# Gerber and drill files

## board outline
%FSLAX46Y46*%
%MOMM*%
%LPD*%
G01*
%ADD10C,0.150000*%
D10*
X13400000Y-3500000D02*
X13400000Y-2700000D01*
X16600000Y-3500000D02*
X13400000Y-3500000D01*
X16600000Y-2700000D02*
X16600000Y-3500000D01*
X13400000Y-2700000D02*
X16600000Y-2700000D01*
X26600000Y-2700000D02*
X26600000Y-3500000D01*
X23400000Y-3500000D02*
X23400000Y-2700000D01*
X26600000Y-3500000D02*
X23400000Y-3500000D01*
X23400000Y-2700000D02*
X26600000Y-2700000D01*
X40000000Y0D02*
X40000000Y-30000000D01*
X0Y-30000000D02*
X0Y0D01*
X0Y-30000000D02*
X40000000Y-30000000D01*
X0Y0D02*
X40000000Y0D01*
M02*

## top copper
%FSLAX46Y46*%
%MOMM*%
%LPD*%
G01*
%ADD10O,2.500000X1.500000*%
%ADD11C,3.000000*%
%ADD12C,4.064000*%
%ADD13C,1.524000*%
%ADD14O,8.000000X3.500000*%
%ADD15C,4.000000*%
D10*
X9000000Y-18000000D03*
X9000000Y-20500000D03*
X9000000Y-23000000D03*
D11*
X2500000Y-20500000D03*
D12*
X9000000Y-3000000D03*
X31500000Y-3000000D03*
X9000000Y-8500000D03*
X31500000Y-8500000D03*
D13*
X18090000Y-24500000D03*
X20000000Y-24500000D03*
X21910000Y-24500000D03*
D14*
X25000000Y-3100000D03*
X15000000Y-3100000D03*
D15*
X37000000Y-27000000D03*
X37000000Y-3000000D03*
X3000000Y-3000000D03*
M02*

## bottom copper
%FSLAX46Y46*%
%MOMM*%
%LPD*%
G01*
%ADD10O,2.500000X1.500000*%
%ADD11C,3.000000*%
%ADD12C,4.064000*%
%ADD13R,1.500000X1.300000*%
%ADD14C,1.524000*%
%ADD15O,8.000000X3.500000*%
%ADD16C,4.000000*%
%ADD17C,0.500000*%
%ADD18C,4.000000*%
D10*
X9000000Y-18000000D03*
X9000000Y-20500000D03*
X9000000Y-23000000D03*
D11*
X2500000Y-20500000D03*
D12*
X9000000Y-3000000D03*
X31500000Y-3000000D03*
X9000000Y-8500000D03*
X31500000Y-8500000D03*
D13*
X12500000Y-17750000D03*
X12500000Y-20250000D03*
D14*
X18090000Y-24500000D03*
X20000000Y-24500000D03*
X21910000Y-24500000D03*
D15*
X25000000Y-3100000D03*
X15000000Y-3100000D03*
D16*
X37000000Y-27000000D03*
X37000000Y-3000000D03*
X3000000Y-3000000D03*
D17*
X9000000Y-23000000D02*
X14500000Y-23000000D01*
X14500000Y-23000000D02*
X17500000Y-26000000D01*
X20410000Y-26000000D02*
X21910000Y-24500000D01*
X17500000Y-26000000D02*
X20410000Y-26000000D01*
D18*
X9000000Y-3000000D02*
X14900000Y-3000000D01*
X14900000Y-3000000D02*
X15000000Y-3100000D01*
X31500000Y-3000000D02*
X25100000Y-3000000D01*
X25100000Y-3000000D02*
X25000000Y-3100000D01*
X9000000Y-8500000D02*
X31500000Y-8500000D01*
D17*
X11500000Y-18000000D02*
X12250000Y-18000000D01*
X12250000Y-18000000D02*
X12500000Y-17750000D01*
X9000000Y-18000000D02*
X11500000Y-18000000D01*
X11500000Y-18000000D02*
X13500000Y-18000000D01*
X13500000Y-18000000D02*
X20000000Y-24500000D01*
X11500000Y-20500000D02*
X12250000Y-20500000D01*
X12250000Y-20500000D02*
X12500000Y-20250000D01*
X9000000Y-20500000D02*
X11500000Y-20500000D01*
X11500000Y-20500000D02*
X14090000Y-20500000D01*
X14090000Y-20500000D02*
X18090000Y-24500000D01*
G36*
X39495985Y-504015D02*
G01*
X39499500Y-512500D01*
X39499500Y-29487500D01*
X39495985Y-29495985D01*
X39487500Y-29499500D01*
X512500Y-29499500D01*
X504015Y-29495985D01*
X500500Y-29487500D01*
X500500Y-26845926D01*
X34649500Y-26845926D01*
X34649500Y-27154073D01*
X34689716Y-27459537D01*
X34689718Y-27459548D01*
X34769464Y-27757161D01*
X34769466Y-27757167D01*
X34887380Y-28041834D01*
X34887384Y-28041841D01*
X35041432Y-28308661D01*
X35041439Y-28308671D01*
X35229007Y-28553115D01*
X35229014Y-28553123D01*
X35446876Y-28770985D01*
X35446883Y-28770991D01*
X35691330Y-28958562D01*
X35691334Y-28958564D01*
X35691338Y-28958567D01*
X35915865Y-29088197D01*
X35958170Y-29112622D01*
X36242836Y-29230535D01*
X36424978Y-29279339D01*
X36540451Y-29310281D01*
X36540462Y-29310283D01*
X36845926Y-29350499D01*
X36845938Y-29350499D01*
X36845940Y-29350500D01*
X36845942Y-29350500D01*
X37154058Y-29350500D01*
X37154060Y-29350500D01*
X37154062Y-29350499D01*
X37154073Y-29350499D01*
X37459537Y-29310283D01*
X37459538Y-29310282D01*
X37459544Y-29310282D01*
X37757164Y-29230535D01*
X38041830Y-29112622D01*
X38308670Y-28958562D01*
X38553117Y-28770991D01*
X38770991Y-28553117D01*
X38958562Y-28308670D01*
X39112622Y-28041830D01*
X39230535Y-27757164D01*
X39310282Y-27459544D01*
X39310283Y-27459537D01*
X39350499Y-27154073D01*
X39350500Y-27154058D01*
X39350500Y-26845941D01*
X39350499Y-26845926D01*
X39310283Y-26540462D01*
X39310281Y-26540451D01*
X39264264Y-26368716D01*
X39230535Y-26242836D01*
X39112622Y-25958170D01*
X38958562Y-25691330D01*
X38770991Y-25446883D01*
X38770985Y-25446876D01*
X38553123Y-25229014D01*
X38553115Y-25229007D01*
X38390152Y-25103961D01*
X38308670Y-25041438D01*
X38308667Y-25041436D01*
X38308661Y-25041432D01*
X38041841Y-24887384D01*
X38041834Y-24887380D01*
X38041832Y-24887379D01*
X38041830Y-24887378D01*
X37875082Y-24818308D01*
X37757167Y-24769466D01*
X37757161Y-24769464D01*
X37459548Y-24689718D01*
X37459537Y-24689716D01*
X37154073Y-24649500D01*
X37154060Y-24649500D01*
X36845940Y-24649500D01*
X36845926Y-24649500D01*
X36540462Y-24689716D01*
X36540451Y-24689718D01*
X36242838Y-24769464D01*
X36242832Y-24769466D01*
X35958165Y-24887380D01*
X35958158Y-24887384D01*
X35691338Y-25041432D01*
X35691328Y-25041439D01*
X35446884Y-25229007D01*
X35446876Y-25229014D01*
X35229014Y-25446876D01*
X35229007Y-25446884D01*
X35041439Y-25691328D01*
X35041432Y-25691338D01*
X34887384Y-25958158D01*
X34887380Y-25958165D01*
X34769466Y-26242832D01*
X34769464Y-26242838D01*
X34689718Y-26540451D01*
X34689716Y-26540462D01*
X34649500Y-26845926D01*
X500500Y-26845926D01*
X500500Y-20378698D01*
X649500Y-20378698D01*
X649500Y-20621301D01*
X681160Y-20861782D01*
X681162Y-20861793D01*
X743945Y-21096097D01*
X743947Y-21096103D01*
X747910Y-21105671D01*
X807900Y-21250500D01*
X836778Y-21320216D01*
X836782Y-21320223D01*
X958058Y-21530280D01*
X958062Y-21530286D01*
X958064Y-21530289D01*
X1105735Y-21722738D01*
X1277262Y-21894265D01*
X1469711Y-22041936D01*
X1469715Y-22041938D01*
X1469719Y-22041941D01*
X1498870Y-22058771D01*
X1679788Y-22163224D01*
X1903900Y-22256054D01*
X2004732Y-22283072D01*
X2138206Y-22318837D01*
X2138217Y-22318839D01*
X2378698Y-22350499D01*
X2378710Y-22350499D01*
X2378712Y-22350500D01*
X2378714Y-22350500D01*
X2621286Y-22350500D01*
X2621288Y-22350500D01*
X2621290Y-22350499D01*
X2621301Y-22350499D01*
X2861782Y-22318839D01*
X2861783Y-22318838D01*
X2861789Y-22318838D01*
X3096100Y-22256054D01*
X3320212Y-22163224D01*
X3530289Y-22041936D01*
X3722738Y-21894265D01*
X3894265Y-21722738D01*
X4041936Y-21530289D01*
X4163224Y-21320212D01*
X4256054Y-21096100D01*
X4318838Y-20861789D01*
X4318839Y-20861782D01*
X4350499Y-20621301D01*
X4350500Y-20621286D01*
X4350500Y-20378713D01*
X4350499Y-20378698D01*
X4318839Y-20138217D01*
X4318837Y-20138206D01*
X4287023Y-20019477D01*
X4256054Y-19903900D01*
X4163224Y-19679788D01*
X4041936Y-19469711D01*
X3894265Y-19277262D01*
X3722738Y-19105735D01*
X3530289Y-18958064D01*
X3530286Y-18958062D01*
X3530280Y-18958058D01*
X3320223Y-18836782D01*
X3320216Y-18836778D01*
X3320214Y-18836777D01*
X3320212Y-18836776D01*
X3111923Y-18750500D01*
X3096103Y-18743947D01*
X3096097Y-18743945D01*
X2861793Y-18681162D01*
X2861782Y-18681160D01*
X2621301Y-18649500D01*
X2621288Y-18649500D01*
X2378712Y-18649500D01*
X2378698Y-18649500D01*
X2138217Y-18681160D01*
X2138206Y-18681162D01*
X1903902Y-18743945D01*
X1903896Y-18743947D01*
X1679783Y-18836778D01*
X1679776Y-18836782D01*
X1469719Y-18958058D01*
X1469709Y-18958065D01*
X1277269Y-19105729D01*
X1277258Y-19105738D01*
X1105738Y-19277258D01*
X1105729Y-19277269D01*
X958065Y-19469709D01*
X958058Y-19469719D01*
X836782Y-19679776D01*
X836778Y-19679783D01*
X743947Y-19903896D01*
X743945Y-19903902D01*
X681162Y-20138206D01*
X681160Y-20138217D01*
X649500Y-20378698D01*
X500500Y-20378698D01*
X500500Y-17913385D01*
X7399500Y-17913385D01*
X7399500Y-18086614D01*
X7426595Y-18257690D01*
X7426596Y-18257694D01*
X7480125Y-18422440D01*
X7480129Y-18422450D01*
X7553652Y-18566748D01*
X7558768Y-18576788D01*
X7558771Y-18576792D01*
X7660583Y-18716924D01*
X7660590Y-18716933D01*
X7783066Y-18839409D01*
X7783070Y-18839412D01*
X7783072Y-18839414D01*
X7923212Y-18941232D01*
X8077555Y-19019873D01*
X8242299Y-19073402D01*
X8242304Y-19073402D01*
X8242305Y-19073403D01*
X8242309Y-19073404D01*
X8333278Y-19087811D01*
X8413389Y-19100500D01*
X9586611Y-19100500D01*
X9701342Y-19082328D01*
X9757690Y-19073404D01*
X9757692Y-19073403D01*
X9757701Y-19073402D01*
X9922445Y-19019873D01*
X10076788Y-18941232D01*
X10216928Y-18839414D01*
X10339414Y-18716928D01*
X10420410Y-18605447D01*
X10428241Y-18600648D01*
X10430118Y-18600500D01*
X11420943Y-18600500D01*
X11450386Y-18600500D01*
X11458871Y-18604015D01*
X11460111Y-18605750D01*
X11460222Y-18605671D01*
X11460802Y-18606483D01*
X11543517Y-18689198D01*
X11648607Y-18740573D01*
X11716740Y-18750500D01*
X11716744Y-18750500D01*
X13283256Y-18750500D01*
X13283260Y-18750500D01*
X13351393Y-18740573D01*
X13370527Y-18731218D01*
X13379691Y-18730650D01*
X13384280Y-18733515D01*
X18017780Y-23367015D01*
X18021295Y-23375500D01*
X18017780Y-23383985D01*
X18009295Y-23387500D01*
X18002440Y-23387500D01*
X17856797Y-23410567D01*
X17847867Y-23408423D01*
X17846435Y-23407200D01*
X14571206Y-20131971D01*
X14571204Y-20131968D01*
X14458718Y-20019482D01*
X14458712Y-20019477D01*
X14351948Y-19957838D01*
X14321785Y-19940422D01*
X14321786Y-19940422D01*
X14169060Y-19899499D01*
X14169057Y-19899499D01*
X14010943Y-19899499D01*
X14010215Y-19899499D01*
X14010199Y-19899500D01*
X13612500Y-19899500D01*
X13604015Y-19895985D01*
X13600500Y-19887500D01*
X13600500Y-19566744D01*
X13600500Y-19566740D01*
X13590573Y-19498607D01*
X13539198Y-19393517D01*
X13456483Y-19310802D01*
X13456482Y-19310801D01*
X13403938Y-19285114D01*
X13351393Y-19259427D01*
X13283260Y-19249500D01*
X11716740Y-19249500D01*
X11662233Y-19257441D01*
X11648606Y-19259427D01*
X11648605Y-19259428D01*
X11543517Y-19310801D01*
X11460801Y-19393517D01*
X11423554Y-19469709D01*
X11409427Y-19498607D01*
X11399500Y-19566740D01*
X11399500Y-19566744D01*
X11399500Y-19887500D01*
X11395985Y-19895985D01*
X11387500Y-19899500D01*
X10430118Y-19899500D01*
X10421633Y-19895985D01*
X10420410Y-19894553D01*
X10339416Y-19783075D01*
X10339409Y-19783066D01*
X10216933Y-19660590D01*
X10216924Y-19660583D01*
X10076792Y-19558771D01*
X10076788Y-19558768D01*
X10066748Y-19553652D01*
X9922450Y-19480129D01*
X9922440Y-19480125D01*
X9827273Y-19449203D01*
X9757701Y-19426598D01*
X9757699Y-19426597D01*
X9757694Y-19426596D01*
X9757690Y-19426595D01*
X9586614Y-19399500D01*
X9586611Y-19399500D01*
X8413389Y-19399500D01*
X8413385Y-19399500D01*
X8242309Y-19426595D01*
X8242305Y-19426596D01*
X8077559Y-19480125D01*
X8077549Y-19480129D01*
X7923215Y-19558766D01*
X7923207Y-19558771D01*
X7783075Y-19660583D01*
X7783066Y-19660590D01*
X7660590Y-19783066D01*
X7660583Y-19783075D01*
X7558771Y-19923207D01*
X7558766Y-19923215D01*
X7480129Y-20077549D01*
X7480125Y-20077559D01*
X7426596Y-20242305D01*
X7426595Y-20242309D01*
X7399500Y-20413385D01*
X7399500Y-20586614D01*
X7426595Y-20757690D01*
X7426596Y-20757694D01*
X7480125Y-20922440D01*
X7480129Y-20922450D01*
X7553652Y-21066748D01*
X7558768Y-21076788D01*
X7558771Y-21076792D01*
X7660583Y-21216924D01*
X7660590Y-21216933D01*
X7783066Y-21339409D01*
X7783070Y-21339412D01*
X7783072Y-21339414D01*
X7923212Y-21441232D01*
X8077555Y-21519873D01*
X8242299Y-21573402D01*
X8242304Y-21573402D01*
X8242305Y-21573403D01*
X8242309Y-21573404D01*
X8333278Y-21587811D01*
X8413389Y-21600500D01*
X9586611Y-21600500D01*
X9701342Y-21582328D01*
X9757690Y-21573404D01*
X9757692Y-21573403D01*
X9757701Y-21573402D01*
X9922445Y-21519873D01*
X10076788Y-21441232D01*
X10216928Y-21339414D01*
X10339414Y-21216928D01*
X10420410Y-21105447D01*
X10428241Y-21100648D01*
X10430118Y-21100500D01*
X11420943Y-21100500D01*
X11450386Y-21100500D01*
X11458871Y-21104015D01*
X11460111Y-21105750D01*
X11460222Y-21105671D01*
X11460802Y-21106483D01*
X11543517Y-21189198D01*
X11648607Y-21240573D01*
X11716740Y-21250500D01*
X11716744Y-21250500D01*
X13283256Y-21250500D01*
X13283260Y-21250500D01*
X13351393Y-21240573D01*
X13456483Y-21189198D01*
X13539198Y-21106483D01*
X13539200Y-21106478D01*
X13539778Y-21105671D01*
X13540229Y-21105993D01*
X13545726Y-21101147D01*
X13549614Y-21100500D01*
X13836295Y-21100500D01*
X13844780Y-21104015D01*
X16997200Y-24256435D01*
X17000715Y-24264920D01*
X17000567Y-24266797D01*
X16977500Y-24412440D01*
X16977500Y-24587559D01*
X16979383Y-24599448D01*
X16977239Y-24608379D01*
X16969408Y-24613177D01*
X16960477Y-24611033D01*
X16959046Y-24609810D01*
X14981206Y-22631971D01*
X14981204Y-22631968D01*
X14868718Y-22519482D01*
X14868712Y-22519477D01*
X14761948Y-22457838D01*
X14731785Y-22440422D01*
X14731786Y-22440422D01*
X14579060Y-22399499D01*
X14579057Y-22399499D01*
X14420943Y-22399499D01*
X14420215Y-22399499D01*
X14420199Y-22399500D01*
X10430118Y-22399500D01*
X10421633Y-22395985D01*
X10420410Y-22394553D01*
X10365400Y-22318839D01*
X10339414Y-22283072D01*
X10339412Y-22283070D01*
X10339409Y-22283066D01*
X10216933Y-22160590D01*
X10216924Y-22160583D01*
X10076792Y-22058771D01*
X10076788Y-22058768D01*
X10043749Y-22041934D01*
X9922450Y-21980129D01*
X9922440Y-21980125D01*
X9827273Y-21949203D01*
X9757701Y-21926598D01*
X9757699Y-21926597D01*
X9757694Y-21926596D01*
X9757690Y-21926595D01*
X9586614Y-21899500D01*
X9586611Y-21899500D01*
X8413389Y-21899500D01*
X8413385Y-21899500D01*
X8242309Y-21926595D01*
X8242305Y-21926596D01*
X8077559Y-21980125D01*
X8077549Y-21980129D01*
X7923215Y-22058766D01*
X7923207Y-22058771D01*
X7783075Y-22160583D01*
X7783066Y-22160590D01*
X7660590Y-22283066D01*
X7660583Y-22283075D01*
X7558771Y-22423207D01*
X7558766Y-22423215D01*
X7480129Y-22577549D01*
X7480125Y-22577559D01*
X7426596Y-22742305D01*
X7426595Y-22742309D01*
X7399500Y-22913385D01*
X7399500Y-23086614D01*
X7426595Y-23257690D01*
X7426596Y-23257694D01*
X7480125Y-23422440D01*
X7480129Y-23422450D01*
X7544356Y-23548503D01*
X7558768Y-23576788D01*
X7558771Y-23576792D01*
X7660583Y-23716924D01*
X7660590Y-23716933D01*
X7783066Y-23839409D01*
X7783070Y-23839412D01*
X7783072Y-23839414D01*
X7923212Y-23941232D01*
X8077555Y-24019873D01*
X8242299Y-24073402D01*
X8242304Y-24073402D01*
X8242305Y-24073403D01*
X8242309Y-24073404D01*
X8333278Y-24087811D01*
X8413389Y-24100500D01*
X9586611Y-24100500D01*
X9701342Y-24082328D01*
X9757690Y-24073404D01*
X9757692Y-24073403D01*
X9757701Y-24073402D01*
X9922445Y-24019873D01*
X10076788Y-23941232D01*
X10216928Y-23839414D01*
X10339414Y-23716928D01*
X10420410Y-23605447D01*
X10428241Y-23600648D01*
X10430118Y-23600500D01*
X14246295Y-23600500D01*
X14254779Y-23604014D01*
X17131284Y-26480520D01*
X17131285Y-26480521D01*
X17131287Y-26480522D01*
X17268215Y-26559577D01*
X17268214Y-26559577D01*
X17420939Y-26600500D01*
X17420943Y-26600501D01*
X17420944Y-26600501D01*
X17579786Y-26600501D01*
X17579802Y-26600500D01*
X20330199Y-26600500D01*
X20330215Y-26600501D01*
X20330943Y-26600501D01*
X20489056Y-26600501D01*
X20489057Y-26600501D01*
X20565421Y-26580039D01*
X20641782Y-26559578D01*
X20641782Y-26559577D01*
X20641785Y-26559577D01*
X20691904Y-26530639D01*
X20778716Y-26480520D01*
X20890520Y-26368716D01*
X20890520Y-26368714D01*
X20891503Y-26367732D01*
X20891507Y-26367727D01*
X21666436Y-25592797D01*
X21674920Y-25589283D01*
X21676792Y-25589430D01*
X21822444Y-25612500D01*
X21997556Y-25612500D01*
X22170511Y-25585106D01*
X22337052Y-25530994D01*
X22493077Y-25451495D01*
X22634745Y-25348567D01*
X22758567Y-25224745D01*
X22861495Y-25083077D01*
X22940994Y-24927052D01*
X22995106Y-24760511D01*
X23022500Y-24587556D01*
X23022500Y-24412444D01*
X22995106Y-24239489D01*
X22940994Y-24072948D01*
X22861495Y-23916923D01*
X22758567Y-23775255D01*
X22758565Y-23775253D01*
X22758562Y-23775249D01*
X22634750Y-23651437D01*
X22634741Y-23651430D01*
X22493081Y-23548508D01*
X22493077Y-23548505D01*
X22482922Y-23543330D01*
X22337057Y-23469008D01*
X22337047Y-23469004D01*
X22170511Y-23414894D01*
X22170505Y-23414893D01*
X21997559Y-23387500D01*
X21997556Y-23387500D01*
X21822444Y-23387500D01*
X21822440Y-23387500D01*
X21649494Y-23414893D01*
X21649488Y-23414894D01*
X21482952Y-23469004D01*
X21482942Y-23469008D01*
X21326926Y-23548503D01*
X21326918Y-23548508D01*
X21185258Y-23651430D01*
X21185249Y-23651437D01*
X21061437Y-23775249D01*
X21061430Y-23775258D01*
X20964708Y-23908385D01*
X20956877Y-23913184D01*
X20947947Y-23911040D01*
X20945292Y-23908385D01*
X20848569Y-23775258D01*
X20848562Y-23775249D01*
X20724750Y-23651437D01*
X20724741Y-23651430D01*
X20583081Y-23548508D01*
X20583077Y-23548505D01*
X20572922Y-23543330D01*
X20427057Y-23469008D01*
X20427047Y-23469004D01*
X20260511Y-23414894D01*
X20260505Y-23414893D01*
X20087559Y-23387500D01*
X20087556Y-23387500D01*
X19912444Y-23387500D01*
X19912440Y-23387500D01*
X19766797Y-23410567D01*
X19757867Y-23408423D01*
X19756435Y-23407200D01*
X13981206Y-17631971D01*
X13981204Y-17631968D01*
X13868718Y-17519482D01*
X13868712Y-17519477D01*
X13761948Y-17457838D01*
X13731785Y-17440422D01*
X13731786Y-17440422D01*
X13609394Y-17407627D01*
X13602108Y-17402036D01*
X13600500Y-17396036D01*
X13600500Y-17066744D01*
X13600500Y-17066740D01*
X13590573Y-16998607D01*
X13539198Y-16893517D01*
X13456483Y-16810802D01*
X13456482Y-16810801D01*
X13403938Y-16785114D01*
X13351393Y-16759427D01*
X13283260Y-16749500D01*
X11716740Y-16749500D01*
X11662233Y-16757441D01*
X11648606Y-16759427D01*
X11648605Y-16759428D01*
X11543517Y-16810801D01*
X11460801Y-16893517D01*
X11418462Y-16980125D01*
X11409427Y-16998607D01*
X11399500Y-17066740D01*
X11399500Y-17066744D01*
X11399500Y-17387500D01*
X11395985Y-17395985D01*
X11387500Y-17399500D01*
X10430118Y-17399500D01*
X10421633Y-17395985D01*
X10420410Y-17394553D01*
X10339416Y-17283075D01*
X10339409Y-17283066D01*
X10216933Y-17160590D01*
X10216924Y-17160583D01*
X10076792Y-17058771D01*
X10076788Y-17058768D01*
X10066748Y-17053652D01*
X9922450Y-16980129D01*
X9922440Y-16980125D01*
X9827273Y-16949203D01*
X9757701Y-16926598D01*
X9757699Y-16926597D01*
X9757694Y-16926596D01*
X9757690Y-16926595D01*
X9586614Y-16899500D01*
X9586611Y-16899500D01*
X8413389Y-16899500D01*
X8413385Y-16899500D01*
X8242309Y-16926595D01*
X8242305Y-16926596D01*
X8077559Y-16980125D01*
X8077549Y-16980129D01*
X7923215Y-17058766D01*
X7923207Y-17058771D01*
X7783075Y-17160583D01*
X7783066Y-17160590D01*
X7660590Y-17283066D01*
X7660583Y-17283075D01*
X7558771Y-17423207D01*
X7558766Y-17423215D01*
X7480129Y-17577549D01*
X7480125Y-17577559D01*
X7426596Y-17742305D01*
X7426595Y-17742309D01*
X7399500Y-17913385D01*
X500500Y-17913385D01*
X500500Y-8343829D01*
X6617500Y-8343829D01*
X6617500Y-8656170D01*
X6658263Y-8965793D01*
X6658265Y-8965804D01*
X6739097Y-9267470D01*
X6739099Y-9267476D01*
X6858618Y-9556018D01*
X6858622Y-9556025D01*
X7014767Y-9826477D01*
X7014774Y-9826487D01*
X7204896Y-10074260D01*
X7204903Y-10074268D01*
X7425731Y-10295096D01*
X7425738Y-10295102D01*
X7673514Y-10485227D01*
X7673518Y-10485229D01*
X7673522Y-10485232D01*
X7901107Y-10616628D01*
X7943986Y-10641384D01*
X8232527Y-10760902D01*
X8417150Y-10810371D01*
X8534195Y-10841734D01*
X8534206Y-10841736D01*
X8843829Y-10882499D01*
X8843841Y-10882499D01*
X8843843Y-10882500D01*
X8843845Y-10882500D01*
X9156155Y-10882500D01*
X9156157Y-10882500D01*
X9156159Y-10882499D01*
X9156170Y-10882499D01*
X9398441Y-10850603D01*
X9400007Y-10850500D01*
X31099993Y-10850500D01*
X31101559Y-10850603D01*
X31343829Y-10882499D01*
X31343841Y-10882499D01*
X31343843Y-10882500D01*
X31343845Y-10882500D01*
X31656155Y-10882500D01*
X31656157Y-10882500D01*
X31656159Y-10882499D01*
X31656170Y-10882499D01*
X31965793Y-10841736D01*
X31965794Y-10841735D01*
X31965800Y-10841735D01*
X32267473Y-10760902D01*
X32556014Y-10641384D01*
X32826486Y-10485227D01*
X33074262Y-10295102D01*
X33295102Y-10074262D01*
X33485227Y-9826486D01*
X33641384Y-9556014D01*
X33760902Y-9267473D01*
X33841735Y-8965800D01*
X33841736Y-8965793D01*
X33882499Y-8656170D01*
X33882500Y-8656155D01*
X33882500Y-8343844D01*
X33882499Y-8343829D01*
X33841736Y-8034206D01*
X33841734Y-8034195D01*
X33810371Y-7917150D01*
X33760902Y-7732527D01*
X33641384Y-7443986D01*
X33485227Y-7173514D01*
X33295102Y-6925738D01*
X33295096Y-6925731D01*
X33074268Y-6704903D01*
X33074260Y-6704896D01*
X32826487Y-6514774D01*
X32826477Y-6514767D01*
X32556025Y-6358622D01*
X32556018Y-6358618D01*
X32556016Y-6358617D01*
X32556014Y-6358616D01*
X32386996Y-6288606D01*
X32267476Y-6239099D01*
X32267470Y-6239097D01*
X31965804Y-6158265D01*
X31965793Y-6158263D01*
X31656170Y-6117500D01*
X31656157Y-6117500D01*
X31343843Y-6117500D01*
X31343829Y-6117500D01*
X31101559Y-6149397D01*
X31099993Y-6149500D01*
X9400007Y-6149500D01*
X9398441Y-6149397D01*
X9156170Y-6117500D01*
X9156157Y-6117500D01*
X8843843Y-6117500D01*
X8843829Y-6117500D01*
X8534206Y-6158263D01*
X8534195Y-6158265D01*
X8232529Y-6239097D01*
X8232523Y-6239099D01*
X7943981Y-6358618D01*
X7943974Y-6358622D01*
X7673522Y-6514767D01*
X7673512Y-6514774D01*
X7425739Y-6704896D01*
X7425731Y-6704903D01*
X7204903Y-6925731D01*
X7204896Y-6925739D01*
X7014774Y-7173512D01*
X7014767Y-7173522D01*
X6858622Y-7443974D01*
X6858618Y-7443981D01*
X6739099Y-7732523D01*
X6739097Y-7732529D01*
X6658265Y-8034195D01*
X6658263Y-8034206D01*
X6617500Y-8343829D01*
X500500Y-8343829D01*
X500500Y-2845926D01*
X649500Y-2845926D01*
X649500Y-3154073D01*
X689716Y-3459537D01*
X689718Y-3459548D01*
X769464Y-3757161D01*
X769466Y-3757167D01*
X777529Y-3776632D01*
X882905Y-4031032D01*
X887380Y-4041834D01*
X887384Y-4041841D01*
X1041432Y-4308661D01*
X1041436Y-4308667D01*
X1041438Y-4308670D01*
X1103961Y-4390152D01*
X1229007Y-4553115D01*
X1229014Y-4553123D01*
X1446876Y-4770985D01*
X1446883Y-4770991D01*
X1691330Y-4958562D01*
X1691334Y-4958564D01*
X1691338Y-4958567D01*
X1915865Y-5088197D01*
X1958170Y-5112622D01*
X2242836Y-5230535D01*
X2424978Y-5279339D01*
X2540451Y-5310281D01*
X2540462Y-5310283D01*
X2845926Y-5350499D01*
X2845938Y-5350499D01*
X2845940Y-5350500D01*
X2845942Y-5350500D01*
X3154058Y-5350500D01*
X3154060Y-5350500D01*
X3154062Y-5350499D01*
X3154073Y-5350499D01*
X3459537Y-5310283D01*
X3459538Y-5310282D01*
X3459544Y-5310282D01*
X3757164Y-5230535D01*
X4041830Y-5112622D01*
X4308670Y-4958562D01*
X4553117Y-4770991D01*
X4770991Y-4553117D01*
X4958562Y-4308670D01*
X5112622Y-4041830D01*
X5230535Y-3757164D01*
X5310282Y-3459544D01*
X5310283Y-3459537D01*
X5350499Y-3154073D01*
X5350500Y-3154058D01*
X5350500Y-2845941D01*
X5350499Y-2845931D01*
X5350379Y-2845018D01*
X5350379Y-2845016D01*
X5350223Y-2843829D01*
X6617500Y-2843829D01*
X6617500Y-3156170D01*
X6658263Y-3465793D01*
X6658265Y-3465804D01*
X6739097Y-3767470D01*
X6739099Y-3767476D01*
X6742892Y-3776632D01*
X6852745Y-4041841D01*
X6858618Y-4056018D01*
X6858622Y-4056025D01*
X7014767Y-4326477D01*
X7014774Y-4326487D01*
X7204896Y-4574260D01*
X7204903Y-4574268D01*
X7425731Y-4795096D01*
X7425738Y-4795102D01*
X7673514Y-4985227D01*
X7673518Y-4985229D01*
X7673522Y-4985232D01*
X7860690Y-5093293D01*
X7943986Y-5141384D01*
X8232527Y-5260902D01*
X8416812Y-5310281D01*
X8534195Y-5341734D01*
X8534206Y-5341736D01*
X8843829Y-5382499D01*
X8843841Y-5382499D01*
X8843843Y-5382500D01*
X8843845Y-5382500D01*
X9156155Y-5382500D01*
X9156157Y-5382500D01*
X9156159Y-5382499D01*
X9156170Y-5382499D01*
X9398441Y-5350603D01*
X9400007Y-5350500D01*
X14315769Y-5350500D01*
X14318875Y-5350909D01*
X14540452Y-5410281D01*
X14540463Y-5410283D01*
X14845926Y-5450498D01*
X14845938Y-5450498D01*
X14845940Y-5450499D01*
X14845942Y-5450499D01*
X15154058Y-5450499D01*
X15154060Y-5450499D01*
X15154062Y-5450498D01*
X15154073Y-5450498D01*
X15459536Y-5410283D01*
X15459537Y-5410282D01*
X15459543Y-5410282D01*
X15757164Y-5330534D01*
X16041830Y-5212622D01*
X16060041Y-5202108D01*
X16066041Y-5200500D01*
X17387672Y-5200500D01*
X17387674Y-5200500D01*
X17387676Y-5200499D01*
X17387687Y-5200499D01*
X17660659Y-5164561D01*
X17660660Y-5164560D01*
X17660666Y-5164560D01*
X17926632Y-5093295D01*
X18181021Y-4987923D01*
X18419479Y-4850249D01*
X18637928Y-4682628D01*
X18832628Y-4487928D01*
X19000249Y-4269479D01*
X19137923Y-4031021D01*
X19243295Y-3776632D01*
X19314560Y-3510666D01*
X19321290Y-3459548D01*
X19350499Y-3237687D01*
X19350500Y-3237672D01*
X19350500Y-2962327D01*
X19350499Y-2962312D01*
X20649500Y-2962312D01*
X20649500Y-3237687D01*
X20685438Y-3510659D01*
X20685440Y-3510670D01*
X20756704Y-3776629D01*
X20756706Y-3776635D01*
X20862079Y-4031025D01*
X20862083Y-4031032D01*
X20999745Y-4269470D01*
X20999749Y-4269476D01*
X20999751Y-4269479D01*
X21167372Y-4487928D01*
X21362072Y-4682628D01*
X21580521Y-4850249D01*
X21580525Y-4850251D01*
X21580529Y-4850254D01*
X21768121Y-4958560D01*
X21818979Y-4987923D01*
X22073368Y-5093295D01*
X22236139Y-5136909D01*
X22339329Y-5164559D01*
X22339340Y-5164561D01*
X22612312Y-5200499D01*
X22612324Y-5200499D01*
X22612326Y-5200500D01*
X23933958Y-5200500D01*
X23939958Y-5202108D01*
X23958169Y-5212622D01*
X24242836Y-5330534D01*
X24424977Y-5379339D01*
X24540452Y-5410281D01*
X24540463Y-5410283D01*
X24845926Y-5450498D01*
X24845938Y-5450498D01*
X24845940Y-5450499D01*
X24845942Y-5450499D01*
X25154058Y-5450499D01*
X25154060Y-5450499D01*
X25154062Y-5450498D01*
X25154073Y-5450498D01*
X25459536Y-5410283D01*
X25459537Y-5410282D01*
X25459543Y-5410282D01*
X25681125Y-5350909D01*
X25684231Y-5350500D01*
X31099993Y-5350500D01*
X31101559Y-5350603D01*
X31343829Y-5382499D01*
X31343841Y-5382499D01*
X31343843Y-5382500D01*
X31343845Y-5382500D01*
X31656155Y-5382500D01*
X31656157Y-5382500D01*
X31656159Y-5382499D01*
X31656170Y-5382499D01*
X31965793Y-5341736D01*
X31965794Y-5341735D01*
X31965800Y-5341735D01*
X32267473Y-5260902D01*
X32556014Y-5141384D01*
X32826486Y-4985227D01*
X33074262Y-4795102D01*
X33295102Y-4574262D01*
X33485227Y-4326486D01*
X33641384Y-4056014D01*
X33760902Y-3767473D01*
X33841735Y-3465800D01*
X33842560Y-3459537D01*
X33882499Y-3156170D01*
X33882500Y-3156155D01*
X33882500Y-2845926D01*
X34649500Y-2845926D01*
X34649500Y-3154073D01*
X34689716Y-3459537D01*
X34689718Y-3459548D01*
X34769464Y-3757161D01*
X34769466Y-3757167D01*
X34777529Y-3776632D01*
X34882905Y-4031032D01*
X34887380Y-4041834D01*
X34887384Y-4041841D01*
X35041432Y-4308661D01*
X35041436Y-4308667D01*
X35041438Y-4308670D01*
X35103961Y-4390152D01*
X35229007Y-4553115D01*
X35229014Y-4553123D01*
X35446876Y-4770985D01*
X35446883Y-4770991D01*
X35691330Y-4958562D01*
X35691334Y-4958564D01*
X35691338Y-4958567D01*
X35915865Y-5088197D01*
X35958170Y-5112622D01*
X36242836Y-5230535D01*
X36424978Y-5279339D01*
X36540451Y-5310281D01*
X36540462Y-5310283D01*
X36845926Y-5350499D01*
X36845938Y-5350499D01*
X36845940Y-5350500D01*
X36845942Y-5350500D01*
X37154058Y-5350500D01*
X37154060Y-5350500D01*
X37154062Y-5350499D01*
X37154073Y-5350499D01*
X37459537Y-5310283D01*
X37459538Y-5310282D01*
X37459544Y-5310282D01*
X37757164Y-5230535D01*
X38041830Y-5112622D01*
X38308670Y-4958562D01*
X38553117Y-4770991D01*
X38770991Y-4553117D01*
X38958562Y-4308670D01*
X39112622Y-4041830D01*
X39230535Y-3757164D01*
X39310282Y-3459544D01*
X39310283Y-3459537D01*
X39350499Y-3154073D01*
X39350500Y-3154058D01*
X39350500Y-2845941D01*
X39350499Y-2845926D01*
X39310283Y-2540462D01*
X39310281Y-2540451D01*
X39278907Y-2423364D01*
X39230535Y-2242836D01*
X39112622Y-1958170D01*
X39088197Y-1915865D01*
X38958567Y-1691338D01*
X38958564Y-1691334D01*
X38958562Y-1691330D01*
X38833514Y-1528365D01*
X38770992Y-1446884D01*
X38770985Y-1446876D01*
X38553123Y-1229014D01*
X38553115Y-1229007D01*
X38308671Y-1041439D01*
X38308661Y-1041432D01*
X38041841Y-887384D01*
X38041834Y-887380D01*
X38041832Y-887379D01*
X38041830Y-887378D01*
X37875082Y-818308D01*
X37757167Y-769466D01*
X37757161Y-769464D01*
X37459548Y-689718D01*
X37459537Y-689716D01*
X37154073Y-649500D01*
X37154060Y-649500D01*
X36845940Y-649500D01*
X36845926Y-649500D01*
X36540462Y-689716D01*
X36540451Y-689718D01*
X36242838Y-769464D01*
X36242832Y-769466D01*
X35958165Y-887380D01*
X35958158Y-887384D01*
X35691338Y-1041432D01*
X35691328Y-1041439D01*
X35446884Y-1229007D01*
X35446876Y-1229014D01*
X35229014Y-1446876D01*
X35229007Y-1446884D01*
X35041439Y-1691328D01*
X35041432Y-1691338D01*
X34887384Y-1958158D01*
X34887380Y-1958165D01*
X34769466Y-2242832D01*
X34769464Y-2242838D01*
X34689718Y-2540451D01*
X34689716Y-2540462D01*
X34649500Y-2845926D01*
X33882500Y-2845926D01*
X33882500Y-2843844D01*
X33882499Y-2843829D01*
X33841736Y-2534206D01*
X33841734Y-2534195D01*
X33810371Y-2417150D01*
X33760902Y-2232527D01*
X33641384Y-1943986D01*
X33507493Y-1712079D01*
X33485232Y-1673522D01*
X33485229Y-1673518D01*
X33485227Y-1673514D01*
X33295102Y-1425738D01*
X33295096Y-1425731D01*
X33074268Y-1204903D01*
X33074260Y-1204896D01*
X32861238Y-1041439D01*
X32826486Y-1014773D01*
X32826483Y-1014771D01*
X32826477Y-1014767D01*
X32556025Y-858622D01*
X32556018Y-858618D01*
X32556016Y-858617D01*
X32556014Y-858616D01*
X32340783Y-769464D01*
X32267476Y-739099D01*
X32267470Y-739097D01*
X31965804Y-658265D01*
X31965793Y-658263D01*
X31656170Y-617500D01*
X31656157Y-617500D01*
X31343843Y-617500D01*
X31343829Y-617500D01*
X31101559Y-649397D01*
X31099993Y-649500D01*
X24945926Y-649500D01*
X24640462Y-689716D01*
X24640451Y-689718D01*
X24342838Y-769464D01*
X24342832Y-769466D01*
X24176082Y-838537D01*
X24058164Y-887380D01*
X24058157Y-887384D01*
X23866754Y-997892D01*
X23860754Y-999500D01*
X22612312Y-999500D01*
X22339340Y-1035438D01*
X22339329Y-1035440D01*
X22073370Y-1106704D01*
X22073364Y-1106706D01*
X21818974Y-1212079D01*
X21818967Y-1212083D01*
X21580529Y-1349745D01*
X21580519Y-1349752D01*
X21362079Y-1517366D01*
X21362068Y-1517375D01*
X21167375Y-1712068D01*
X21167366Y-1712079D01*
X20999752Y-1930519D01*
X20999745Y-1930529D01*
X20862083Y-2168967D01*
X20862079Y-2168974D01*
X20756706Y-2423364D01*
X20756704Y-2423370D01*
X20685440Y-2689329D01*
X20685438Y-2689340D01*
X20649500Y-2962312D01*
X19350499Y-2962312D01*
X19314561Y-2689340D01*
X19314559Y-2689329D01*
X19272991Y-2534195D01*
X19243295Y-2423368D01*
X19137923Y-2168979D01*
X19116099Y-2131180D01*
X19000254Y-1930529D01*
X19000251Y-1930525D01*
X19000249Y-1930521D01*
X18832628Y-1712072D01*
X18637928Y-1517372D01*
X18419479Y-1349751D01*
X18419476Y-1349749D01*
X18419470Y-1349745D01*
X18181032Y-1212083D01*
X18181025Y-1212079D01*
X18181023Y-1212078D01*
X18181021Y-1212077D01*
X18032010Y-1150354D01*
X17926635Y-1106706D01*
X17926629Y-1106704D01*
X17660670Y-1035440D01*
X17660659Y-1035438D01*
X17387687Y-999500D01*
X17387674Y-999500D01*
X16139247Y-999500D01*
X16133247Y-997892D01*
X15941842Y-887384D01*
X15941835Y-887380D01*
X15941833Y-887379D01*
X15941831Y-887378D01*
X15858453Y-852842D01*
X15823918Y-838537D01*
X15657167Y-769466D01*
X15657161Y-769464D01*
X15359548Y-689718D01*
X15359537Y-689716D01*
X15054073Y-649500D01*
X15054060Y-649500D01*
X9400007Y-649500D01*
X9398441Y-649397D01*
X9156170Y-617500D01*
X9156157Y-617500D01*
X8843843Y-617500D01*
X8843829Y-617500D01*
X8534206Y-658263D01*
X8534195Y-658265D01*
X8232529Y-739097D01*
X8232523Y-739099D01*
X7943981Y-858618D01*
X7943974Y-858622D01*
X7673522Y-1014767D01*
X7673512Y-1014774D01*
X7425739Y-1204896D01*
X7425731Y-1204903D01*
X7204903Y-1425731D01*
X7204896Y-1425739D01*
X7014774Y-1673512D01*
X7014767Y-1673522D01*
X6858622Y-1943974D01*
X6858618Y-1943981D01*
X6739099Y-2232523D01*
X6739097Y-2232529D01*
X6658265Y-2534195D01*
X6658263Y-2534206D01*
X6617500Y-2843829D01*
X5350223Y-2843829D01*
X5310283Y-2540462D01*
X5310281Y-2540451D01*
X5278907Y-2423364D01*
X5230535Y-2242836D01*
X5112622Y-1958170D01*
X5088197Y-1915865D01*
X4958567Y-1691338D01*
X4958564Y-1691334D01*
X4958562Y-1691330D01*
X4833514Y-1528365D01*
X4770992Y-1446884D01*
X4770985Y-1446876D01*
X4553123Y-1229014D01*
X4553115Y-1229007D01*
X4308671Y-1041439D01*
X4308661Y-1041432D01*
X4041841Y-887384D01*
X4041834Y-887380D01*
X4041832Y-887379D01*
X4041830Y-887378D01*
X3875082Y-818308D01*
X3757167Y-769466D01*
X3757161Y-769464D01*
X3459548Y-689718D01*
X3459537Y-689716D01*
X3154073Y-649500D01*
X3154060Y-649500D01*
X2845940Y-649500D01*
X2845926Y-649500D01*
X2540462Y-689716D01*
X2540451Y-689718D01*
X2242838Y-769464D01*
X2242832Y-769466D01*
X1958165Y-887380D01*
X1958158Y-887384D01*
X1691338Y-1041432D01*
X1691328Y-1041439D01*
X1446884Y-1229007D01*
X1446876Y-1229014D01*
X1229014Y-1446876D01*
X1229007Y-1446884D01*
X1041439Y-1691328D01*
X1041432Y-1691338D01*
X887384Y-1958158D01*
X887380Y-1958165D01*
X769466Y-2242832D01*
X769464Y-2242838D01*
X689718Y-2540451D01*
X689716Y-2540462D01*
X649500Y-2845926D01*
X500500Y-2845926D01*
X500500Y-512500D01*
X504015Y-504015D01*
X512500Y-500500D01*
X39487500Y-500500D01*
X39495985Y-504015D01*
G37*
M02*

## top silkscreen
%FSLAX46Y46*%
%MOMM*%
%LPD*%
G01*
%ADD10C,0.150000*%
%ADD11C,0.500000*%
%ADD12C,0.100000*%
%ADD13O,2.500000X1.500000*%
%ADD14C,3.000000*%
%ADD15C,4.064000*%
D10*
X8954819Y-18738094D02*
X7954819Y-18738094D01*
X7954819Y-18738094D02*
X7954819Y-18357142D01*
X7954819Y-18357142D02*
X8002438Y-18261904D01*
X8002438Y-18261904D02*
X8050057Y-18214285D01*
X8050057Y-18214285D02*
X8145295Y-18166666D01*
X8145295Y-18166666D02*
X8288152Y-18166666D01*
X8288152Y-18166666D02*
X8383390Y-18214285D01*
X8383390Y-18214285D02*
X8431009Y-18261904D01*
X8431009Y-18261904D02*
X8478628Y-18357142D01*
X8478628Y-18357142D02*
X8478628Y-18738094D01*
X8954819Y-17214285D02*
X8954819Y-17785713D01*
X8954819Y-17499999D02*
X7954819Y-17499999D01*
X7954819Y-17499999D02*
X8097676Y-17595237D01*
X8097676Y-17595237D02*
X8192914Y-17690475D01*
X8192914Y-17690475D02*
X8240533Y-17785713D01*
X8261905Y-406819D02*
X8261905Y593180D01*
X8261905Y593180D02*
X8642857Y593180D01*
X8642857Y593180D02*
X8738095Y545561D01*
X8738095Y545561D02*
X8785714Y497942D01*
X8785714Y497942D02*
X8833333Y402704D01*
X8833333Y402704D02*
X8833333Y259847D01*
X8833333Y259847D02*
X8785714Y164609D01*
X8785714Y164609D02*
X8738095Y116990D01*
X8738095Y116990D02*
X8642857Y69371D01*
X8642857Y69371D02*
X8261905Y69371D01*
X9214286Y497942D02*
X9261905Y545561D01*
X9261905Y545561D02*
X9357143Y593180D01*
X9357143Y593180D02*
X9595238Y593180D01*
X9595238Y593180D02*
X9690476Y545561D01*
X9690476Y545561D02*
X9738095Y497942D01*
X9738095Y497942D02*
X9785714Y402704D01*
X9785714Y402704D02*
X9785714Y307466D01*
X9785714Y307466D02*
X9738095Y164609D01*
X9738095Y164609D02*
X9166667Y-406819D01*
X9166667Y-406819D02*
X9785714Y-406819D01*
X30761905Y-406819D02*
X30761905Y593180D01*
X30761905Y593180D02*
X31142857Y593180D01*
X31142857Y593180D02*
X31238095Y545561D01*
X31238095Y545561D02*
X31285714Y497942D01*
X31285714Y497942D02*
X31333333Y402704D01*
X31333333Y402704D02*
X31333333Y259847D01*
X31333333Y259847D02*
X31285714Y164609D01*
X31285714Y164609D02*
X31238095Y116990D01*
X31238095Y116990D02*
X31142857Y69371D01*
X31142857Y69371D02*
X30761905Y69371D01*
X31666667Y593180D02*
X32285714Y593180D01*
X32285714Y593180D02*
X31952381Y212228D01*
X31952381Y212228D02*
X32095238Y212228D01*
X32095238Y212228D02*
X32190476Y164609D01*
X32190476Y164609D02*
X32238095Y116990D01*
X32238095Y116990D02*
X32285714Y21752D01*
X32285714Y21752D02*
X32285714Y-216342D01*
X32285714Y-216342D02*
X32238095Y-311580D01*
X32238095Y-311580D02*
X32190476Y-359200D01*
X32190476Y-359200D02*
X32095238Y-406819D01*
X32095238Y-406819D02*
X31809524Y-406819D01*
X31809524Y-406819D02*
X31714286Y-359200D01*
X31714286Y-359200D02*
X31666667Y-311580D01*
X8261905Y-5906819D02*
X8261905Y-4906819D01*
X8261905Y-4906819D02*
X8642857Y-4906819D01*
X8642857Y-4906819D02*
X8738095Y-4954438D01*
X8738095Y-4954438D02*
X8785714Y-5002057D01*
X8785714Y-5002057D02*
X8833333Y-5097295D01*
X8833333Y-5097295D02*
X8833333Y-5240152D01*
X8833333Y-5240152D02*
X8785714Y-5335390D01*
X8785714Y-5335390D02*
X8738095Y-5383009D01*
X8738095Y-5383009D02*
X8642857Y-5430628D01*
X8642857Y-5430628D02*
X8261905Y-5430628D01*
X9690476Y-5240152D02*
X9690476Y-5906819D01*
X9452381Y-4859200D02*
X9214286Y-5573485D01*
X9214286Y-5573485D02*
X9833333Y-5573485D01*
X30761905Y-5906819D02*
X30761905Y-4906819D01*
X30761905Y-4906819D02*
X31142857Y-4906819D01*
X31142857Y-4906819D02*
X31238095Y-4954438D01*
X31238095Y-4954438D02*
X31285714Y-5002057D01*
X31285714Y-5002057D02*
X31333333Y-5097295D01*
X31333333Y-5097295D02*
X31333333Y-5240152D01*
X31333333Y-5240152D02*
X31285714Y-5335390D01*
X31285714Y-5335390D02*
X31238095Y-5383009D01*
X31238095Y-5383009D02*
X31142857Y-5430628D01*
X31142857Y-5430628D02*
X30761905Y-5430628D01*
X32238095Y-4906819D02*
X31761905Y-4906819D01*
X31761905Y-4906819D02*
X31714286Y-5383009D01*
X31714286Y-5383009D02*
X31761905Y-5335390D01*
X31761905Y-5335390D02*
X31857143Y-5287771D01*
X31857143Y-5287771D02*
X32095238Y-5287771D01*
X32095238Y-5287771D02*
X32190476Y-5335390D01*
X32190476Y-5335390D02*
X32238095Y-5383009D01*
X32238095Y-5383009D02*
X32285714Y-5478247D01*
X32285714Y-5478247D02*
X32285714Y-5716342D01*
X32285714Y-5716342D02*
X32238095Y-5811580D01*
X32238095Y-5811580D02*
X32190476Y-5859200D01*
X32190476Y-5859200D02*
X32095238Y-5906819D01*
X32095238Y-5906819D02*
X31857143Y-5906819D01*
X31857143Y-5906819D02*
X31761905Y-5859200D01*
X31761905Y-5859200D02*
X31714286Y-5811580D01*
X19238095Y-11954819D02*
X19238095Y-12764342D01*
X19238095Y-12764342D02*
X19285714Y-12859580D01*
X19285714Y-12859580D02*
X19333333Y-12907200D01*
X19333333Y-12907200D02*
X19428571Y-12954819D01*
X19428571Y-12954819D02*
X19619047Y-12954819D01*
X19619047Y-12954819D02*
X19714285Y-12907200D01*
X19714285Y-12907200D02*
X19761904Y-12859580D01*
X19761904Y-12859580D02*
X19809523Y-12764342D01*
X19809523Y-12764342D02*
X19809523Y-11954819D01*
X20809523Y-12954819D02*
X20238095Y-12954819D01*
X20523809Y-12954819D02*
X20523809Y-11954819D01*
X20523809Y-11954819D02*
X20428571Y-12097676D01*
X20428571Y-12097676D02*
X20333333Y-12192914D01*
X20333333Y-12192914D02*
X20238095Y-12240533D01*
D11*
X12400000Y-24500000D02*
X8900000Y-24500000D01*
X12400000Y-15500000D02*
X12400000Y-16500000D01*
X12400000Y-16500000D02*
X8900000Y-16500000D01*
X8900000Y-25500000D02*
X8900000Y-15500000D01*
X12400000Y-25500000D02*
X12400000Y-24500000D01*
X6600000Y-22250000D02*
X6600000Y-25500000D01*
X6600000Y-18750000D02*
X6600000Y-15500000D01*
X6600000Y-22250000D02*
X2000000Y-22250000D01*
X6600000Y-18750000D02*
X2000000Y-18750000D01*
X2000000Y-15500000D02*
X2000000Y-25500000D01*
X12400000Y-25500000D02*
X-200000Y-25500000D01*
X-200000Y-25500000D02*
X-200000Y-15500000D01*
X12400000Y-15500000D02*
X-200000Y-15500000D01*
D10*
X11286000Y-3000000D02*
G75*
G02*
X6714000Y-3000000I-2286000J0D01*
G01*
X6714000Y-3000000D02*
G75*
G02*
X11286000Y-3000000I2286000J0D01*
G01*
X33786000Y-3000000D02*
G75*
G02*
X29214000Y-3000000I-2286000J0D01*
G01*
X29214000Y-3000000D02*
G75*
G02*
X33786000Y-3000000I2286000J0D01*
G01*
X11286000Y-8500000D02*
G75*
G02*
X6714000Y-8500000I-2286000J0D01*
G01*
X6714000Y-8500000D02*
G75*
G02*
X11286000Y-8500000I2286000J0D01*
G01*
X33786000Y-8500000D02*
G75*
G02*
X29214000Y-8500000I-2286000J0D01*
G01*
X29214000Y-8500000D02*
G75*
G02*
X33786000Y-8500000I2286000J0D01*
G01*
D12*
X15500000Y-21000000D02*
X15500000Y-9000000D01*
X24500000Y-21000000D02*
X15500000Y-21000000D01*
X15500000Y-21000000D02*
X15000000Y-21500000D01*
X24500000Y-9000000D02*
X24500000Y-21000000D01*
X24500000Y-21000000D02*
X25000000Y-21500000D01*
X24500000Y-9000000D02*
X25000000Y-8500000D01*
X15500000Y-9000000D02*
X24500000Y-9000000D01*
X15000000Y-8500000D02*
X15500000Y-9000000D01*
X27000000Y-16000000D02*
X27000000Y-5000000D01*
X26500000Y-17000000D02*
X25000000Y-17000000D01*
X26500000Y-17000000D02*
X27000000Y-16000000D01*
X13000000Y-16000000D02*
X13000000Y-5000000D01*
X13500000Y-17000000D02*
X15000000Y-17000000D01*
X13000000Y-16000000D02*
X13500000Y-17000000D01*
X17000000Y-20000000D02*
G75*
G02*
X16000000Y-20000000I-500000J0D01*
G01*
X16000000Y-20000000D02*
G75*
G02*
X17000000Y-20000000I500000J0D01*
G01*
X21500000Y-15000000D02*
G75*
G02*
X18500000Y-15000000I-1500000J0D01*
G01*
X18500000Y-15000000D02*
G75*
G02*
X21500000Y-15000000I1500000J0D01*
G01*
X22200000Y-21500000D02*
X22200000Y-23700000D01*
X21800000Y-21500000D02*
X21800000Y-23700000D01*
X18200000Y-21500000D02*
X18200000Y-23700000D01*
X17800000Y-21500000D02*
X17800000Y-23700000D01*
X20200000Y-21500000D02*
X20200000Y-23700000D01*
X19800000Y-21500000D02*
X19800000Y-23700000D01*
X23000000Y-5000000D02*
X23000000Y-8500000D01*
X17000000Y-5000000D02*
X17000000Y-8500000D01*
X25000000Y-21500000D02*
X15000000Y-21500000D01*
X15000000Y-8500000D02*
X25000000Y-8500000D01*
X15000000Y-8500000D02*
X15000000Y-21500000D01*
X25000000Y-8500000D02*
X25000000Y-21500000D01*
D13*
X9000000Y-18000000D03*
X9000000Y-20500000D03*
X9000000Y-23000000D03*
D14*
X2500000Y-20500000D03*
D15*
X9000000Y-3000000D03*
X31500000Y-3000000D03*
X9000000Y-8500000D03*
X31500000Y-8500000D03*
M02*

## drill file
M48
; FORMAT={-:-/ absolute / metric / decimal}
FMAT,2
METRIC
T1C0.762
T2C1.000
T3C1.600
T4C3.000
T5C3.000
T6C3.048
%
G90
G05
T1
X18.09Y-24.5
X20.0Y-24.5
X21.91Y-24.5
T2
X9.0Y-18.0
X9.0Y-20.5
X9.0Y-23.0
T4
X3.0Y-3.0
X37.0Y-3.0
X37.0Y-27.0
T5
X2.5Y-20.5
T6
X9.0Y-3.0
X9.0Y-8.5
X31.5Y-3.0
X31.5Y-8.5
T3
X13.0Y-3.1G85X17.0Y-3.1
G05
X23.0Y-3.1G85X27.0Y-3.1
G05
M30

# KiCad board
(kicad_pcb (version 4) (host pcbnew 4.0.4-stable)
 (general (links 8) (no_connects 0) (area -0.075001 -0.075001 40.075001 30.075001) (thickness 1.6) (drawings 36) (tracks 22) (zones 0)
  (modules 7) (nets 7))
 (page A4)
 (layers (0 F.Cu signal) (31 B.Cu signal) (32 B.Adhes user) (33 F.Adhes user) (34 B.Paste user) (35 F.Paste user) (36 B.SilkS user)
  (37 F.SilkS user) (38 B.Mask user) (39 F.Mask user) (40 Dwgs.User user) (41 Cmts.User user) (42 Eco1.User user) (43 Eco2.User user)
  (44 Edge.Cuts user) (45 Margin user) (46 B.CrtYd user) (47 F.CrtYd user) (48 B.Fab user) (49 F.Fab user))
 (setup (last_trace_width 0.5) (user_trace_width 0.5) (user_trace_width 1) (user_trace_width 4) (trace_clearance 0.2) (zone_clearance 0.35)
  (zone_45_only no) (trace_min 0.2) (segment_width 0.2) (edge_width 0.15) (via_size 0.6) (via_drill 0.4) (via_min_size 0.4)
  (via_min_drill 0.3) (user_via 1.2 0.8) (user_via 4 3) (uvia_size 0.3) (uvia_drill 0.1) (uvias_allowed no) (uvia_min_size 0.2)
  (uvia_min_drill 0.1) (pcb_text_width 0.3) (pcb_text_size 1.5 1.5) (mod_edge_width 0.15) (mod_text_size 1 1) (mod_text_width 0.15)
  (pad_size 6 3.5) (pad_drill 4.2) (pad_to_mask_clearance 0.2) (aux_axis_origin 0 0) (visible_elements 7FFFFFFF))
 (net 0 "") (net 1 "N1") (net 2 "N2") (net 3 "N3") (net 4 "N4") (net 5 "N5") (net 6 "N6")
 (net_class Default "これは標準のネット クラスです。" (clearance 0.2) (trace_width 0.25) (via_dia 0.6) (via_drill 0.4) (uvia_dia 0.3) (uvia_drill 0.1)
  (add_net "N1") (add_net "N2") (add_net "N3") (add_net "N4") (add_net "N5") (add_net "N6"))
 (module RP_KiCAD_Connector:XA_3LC (layer F.Cu) (at 9 18 270)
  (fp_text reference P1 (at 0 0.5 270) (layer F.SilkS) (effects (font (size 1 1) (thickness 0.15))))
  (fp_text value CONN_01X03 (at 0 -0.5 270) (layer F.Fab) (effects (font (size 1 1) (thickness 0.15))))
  (fp_line (start 6.5 -3.4) (end 6.5 0.1) (layer F.SilkS) (width 0.5))
  (fp_line (start -2.5 -3.4) (end -1.5 -3.4) (layer F.SilkS) (width 0.5))
  (fp_line (start -1.5 -3.4) (end -1.5 0.1) (layer F.SilkS) (width 0.5))
  (fp_line (start 7.5 0.1) (end -2.5 0.1) (layer F.SilkS) (width 0.5))
  (fp_line (start 7.5 -3.4) (end 6.5 -3.4) (layer F.SilkS) (width 0.5))
  (fp_line (start 4.25 2.4) (end 7.5 2.4) (layer F.SilkS) (width 0.5))
  (fp_line (start 0.75 2.4) (end -2.5 2.4) (layer F.SilkS) (width 0.5))
  (fp_line (start 4.25 2.4) (end 4.25 7) (layer F.SilkS) (width 0.5))
  (fp_line (start 0.75 2.4) (end 0.75 7) (layer F.SilkS) (width 0.5))
  (fp_line (start -2.5 7) (end 7.5 7) (layer F.SilkS) (width 0.5))
  (fp_line (start 7.5 -3.4) (end 7.5 9.2) (layer F.SilkS) (width 0.5))
  (fp_line (start 7.5 9.2) (end -2.5 9.2) (layer F.SilkS) (width 0.5))
  (fp_line (start -2.5 -3.4) (end -2.5 9.2) (layer F.SilkS) (width 0.5))
  (pad 1 thru_hole oval (at 0 0 270) (size 1.5 2.5) (drill 1) (layers *.Cu *.Mask F.SilkS) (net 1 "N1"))
  (pad 2 thru_hole oval (at 2.5 0 270) (size 1.5 2.5) (drill 1) (layers *.Cu *.Mask F.SilkS) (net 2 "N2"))
  (pad 3 thru_hole oval (at 5 0 270) (size 1.5 2.5) (drill 1) (layers *.Cu *.Mask F.SilkS) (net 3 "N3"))
  (pad "" thru_hole circle (at 2.5 6.5 270) (size 3 3) (drill 3) (layers *.Cu *.Mask F.SilkS) (clearance -0.3)))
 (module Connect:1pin (layer F.Cu) (at 9 3)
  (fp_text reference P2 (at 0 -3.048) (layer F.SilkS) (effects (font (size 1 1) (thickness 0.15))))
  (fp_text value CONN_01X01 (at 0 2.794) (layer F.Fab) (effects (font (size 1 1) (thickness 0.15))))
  (fp_circle (center 0 0) (end 0 -2.286) (layer F.SilkS) (width 0.15))
  (pad 1 thru_hole circle (at 0 0) (size 4.064 4.064) (drill 3.048) (layers *.Cu *.Mask F.SilkS) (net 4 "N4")))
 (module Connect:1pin (layer F.Cu) (at 31.5 3)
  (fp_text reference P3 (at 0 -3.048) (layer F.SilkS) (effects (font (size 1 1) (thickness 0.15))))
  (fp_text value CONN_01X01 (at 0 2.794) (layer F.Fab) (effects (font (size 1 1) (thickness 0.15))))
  (fp_circle (center 0 0) (end 0 -2.286) (layer F.SilkS) (width 0.15))
  (pad 1 thru_hole circle (at 0 0) (size 4.064 4.064) (drill 3.048) (layers *.Cu *.Mask F.SilkS) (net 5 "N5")))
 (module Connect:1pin (layer F.Cu) (at 9 8.5)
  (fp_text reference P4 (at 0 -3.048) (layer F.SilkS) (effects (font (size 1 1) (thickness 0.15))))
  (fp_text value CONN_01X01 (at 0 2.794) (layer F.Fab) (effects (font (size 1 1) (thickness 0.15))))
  (fp_circle (center 0 0) (end 0 -2.286) (layer F.SilkS) (width 0.15))
  (pad 1 thru_hole circle (at 0 0) (size 4.064 4.064) (drill 3.048) (layers *.Cu *.Mask F.SilkS) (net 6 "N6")))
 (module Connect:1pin (layer F.Cu) (at 31.5 8.5)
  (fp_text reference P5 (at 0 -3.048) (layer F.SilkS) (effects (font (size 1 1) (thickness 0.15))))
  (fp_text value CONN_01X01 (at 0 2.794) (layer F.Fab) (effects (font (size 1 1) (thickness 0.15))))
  (fp_circle (center 0 0) (end 0 -2.286) (layer F.SilkS) (width 0.15))
  (pad 1 thru_hole circle (at 0 0) (size 4.064 4.064) (drill 3.048) (layers *.Cu *.Mask F.SilkS) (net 6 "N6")))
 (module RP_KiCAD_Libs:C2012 (layer B.Cu) (at 12.5 19 270)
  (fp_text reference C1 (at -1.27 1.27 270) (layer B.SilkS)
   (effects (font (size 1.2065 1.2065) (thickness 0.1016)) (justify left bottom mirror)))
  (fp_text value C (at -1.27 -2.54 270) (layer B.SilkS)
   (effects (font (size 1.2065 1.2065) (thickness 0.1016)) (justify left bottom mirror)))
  (pad 1 smd rect (at -1.25 0 270) (size 1.3 1.5) (layers B.Cu B.Paste B.Mask) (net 1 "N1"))
  (pad 2 smd rect (at 1.25 0 270) (size 1.3 1.5) (layers B.Cu B.Paste B.Mask) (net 2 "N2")))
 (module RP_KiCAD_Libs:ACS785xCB (layer F.Cu) (at 20 24.5)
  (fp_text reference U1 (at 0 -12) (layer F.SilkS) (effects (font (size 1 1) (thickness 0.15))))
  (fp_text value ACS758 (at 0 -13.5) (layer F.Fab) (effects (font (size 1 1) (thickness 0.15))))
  (fp_line (start -4.5 -3.5) (end -4.5 -15.5) (layer F.SilkS) (width 0.1))
  (fp_line (start 4.5 -3.5) (end -4.5 -3.5) (layer F.SilkS) (width 0.1))
  (fp_line (start -4.5 -3.5) (end -5 -3) (layer F.SilkS) (width 0.1))
  (fp_line (start 4.5 -15.5) (end 4.5 -3.5) (layer F.SilkS) (width 0.1))
  (fp_line (start 4.5 -3.5) (end 5 -3) (layer F.SilkS) (width 0.1))
  (fp_line (start 4.5 -15.5) (end 5 -16) (layer F.SilkS) (width 0.1))
  (fp_line (start -4.5 -15.5) (end 4.5 -15.5) (layer F.SilkS) (width 0.1))
  (fp_line (start -5 -16) (end -4.5 -15.5) (layer F.SilkS) (width 0.1))
  (fp_line (start 7 -8.5) (end 7 -19.5) (layer F.SilkS) (width 0.1))
  (fp_line (start 6.5 -7.5) (end 5 -7.5) (layer F.SilkS) (width 0.1))
  (fp_line (start 6.5 -7.5) (end 7 -8.5) (layer F.SilkS) (width 0.1))
  (fp_line (start -7 -8.5) (end -7 -19.5) (layer F.SilkS) (width 0.1))
  (fp_line (start -6.5 -7.5) (end -5 -7.5) (layer F.SilkS) (width 0.1))
  (fp_line (start -7 -8.5) (end -6.5 -7.5) (layer F.SilkS) (width 0.1))
  (fp_circle (center -3.5 -4.5) (end -3 -4.5) (layer F.SilkS) (width 0.1))
  (fp_circle (center 0 -9.5) (end 0 -11) (layer F.SilkS) (width 0.1))
  (fp_line (start 2.2 -3) (end 2.2 -0.8) (layer F.SilkS) (width 0.1))
  (fp_line (start 1.8 -3) (end 1.8 -0.8) (layer F.SilkS) (width 0.1))
  (fp_line (start -1.8 -3) (end -1.8 -0.8) (layer F.SilkS) (width 0.1))
  (fp_line (start -2.2 -3) (end -2.2 -0.8) (layer F.SilkS) (width 0.1))
  (fp_line (start 0.2 -3) (end 0.2 -0.8) (layer F.SilkS) (width 0.1))
  (fp_line (start -0.2 -3) (end -0.2 -0.8) (layer F.SilkS) (width 0.1))
  (fp_line (start 3 -19.5) (end 3 -16) (layer F.SilkS) (width 0.1))
  (fp_line (start -3 -19.5) (end -3 -16) (layer F.SilkS) (width 0.1))
  (fp_line (start 5 -3) (end -5 -3) (layer F.SilkS) (width 0.1))
  (fp_line (start -5 -16) (end 5 -16) (layer F.SilkS) (width 0.1))
  (fp_line (start -5 -16) (end -5 -3) (layer F.SilkS) (width 0.1))
  (fp_line (start 5 -16) (end 5 -3) (layer F.SilkS) (width 0.1))
  (pad 1 thru_hole circle (at -1.91 0) (size 1.524 1.524) (drill 0.762) (layers *.Cu *.Mask) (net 2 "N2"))
  (pad 2 thru_hole circle (at 0 0) (size 1.524 1.524) (drill 0.762) (layers *.Cu *.Mask) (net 1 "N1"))
  (pad 3 thru_hole circle (at 1.91 0) (size 1.524 1.524) (drill 0.762) (layers *.Cu *.Mask) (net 3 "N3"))
  (pad 4 thru_hole oval (at 5 -21.4) (size 8 3.5) (drill oval 5.6 1.6) (layers *.Cu *.Mask) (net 5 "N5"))
  (pad 5 thru_hole oval (at -5 -21.4) (size 8 3.5) (drill oval 5.6 1.6) (layers *.Cu *.Mask) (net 4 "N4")))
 (gr_line (start 13.4 3.5) (end 13.4 2.7) (angle 90) (layer Edge.Cuts) (width 0.15))
 (gr_line (start 16.6 3.5) (end 13.4 3.5) (angle 90) (layer Edge.Cuts) (width 0.15))
 (gr_line (start 16.6 2.7) (end 16.6 3.5) (angle 90) (layer Edge.Cuts) (width 0.15))
 (gr_line (start 13.4 2.7) (end 16.6 2.7) (angle 90) (layer Edge.Cuts) (width 0.15))
 (gr_line (start 26.6 2.7) (end 26.6 3.5) (angle 90) (layer Edge.Cuts) (width 0.15))
 (gr_line (start 23.4 3.5) (end 23.4 2.7) (angle 90) (layer Edge.Cuts) (width 0.15))
 (gr_line (start 26.6 3.5) (end 23.4 3.5) (angle 90) (layer Edge.Cuts) (width 0.15))
 (gr_line (start 23.4 2.7) (end 26.6 2.7) (angle 90) (layer Edge.Cuts) (width 0.15))
 (gr_line (start 40 0) (end 40 30) (angle 90) (layer Edge.Cuts) (width 0.15))
 (gr_line (start 0 30) (end 0 0) (angle 90) (layer Edge.Cuts) (width 0.15))
 (gr_line (start 0 30) (end 40 30) (angle 90) (layer Edge.Cuts) (width 0.15))
 (gr_line (start 0 0) (end 40 0) (angle 90) (layer Edge.Cuts) (width 0.15))
 (via (at 37 27) (size 4) (drill 3) (layers F.Cu B.Cu) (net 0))
 (via (at 37 3) (size 4) (drill 3) (layers F.Cu B.Cu) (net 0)) (via (at 3 3) (size 4) (drill 3) (layers F.Cu B.Cu) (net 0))
 (segment (start 9 23) (end 14.5 23) (width 0.5) (layer B.Cu) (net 3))
 (segment (start 14.5 23) (end 17.5 26) (width 0.5) (layer B.Cu) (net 3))
 (segment (start 20.41 26) (end 21.91 24.5) (width 0.5) (layer B.Cu) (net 3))
 (segment (start 17.5 26) (end 20.41 26) (width 0.5) (layer B.Cu) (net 3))
 (segment (start 9 3) (end 14.9 3) (width 4) (layer B.Cu) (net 4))
 (segment (start 14.9 3) (end 15 3.1) (width 4) (layer B.Cu) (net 4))
 (segment (start 31.5 3) (end 25.1 3) (width 4) (layer B.Cu) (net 5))
 (segment (start 25.1 3) (end 25 3.1) (width 4) (layer B.Cu) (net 5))
 (segment (start 9 8.5) (end 31.5 8.5) (width 4) (layer B.Cu) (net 6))
 (segment (start 11.5 18) (end 12.25 18) (width 0.5) (layer B.Cu) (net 1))
 (segment (start 12.25 18) (end 12.5 17.75) (width 0.5) (layer B.Cu) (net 1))
 (segment (start 9 18) (end 11.5 18) (width 0.5) (layer B.Cu) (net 1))
 (segment (start 11.5 18) (end 13.5 18) (width 0.5) (layer B.Cu) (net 1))
 (segment (start 13.5 18) (end 20 24.5) (width 0.5) (layer B.Cu) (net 1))
 (segment (start 11.5 20.5) (end 12.25 20.5) (width 0.5) (layer B.Cu) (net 2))
 (segment (start 12.25 20.5) (end 12.5 20.25) (width 0.5) (layer B.Cu) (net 2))
 (segment (start 9 20.5) (end 11.5 20.5) (width 0.5) (layer B.Cu) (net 2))
 (segment (start 11.5 20.5) (end 14.09 20.5) (width 0.5) (layer B.Cu) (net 2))
 (segment (start 14.09 20.5) (end 18.09 24.5) (width 0.5) (layer B.Cu) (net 2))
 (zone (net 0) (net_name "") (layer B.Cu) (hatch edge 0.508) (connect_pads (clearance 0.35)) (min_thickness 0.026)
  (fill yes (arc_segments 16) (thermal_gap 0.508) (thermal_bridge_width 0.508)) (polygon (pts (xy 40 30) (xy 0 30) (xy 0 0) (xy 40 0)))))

